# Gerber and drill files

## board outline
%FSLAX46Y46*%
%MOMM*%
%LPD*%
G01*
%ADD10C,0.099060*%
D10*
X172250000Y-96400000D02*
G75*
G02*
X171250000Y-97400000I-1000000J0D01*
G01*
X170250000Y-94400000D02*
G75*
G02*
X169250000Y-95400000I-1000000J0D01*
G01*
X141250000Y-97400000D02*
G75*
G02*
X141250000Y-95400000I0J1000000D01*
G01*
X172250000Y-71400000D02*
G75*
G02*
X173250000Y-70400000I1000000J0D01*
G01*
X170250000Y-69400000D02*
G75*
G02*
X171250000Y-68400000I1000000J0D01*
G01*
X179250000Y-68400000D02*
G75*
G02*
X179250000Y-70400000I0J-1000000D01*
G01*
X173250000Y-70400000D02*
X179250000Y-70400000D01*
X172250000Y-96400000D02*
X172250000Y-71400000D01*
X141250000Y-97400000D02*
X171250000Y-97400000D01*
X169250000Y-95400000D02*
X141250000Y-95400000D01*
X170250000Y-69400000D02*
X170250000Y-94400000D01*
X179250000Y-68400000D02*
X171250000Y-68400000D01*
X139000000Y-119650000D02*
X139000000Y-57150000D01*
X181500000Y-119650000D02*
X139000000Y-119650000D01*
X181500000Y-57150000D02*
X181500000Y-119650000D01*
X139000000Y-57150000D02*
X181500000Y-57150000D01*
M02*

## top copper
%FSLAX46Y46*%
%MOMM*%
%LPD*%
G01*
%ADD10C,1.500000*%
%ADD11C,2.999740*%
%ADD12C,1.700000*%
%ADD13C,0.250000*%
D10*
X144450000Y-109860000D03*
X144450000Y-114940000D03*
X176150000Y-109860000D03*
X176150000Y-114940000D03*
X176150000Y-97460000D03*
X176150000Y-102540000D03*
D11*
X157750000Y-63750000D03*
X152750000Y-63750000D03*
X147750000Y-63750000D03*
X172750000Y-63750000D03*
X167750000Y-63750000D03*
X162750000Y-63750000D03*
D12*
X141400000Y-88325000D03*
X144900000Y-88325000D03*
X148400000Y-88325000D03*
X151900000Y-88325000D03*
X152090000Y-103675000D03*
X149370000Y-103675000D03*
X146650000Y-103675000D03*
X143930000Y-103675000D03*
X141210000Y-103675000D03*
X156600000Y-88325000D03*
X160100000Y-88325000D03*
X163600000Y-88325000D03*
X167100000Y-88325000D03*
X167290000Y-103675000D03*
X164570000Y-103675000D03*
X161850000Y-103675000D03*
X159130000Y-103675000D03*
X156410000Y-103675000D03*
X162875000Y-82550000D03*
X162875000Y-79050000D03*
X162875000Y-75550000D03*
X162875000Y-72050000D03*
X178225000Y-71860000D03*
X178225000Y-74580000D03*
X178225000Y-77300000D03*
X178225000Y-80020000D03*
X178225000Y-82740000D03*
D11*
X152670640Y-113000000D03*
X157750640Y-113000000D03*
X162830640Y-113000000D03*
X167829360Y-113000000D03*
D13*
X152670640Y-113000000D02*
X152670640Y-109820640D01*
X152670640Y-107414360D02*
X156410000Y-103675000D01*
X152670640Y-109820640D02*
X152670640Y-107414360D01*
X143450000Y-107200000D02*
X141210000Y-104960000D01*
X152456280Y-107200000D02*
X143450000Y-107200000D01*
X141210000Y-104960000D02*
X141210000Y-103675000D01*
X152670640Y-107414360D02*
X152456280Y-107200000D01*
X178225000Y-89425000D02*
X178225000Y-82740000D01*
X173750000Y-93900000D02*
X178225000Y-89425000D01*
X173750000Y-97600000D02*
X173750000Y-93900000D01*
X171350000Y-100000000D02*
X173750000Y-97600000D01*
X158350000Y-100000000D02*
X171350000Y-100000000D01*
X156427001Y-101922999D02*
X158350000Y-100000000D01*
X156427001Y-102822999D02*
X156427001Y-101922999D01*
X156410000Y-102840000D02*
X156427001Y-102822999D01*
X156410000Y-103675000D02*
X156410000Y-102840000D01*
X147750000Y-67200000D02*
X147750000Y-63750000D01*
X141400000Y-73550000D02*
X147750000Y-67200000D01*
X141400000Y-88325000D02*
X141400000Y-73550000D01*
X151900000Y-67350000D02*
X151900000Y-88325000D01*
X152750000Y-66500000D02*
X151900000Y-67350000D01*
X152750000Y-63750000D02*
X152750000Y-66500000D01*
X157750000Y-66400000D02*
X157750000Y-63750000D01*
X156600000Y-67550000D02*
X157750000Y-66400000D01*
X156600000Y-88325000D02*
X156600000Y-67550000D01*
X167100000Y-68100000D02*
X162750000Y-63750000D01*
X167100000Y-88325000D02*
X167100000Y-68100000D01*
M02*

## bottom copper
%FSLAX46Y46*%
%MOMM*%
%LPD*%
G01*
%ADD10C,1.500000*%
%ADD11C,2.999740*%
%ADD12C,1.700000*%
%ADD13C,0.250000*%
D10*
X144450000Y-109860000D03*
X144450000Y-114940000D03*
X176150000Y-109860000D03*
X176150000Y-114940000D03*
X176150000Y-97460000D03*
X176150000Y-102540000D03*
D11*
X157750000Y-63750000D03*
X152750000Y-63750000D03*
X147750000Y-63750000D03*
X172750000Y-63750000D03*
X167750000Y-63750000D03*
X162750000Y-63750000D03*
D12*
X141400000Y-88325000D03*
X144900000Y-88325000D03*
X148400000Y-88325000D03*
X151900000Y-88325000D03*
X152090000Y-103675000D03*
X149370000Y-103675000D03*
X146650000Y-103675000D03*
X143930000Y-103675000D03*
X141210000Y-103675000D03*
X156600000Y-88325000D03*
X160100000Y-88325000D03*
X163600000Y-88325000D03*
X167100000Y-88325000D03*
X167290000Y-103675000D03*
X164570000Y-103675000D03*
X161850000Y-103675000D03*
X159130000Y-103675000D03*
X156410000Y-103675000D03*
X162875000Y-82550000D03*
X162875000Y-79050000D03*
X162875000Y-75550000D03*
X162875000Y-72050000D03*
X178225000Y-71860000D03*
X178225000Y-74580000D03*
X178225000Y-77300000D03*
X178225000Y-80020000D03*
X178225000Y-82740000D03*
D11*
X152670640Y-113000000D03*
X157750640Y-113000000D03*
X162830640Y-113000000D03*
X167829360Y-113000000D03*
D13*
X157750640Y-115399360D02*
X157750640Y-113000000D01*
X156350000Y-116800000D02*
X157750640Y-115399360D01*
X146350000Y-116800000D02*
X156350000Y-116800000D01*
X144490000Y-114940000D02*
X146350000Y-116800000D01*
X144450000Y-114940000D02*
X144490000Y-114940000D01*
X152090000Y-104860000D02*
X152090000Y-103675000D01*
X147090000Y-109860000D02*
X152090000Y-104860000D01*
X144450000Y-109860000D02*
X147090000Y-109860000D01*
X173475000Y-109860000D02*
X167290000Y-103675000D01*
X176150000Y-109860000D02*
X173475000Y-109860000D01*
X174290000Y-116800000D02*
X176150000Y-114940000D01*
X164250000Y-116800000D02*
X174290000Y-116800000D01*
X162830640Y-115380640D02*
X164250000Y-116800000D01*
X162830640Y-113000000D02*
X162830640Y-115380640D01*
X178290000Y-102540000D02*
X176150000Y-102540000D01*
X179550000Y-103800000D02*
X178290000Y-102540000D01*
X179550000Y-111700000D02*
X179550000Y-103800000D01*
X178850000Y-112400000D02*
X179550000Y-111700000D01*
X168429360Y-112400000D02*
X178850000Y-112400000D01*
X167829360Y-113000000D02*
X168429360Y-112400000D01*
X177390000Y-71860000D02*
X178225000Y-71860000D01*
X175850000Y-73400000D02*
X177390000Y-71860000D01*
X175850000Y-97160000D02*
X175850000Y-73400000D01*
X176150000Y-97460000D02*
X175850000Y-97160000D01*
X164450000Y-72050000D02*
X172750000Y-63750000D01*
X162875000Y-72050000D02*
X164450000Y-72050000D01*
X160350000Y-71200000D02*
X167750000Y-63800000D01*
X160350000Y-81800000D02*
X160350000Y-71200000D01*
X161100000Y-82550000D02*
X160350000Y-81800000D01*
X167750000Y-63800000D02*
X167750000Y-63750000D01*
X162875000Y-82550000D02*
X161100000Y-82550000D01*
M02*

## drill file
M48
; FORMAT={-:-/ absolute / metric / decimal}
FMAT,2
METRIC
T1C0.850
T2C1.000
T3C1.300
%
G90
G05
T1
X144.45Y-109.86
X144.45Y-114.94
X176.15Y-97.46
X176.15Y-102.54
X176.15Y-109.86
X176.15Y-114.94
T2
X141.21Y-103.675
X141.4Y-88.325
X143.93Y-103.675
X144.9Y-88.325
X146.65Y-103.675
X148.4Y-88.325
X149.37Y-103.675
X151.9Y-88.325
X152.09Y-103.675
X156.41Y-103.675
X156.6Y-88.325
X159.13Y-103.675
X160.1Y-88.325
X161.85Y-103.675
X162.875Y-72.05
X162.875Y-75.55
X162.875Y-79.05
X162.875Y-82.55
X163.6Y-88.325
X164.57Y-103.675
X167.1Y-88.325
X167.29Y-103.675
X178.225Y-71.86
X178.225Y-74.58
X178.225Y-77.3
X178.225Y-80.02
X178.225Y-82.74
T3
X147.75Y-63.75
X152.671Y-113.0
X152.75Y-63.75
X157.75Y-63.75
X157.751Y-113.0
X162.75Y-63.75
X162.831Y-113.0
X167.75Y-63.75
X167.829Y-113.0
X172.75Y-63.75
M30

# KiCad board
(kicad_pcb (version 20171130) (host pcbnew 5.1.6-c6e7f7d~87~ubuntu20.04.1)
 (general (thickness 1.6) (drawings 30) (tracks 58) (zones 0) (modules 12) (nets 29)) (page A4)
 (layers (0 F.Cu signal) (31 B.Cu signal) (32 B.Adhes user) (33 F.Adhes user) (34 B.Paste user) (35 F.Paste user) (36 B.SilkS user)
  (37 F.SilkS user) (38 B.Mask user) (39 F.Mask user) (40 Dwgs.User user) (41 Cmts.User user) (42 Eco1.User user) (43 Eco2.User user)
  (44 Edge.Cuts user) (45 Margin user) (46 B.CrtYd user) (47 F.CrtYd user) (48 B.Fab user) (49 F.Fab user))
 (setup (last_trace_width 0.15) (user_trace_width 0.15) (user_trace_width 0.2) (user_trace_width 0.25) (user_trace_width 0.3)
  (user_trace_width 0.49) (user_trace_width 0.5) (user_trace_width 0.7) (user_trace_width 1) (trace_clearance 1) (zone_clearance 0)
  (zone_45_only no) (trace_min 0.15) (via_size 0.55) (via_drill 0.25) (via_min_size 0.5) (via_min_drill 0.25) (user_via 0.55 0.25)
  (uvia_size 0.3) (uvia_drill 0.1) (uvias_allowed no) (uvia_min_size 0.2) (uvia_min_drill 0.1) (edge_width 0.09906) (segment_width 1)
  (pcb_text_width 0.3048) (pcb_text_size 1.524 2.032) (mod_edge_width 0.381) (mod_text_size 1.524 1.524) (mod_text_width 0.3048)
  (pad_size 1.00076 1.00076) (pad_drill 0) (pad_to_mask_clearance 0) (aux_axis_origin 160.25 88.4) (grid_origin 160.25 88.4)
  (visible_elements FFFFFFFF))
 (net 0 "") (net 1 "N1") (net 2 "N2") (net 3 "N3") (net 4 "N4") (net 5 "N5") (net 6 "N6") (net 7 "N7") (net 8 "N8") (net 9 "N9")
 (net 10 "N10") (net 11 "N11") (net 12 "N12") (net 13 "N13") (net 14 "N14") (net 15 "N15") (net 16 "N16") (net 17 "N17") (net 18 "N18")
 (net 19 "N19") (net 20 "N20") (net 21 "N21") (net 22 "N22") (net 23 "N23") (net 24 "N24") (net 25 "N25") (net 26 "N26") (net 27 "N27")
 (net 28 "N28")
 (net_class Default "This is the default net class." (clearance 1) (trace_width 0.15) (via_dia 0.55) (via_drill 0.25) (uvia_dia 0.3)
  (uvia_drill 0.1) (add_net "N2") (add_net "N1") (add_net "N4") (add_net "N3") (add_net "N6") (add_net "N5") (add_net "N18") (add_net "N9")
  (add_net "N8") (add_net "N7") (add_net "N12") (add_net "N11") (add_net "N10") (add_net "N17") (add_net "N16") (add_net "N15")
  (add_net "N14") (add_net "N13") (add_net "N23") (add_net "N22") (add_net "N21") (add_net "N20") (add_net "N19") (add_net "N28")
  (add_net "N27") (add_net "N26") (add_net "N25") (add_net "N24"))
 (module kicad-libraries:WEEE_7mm (layer B.Cu) (at 148.85 80.5 180)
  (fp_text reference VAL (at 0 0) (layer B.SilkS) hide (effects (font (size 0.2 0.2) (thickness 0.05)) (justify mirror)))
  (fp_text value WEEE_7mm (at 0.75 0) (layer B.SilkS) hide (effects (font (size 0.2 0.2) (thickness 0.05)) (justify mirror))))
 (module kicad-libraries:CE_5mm (layer B.Cu) (at 148.95 73.1 180)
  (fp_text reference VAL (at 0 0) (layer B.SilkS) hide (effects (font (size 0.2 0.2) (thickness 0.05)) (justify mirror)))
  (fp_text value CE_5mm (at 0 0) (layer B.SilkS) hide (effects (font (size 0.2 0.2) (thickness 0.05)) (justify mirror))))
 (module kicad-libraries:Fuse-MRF (layer F.Cu) (at 144.45 112.4 90)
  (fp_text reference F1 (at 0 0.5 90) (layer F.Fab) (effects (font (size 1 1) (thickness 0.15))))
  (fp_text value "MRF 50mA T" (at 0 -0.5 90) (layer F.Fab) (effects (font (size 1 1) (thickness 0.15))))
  (pad 2 thru_hole circle (at 2.54 0 90) (size 1.5 1.5) (drill 0.85) (layers *.Cu *.Mask) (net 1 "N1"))
  (pad 1 thru_hole circle (at -2.54 0 90) (size 1.5 1.5) (drill 0.85) (layers *.Cu *.Mask) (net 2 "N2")))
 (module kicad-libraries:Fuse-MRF (layer F.Cu) (at 176.15 112.4 90)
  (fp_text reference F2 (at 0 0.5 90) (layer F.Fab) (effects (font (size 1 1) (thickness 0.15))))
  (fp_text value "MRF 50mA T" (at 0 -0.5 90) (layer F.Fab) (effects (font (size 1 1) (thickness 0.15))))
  (pad 2 thru_hole circle (at 2.54 0 90) (size 1.5 1.5) (drill 0.85) (layers *.Cu *.Mask) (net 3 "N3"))
  (pad 1 thru_hole circle (at -2.54 0 90) (size 1.5 1.5) (drill 0.85) (layers *.Cu *.Mask) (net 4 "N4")))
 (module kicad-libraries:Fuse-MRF (layer F.Cu) (at 176.15 100 90)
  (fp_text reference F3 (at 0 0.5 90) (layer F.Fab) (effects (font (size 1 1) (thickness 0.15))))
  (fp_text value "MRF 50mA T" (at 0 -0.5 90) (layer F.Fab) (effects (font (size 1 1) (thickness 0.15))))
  (pad 2 thru_hole circle (at 2.54 0 90) (size 1.5 1.5) (drill 0.85) (layers *.Cu *.Mask) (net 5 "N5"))
  (pad 1 thru_hole circle (at -2.54 0 90) (size 1.5 1.5) (drill 0.85) (layers *.Cu *.Mask) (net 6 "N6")))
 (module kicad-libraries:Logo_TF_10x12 (layer F.Cu) (at 149.25 74.4)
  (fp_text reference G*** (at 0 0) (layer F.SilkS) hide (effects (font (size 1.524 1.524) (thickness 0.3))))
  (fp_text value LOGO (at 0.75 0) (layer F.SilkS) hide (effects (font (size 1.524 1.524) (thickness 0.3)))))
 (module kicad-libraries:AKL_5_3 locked (layer F.Cu) (at 152.75 63.75)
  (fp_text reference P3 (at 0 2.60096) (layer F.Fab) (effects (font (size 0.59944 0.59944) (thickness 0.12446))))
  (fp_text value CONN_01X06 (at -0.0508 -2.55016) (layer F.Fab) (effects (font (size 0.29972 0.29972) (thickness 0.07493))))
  (pad 3 thru_hole circle (at 5 0) (size 2.99974 2.99974) (drill 1.30048) (layers *.Cu *.Mask F.SilkS) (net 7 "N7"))
  (pad 2 thru_hole circle (at 0 0) (size 2.99974 2.99974) (drill 1.30048) (layers *.Cu *.Mask F.SilkS) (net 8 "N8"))
  (pad 1 thru_hole circle (at -5 0) (size 2.99974 2.99974) (drill 1.30048) (layers *.Cu *.Mask F.SilkS) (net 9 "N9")))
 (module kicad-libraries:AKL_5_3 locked (layer F.Cu) (at 167.75 63.75)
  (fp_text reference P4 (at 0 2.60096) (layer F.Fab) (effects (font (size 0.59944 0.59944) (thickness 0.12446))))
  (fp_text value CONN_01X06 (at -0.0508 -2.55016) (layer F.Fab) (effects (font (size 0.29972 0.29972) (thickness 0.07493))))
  (pad 3 thru_hole circle (at 5 0) (size 2.99974 2.99974) (drill 1.30048) (layers *.Cu *.Mask F.SilkS) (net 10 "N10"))
  (pad 2 thru_hole circle (at 0 0) (size 2.99974 2.99974) (drill 1.30048) (layers *.Cu *.Mask F.SilkS) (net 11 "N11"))
  (pad 1 thru_hole circle (at -5 0) (size 2.99974 2.99974) (drill 1.30048) (layers *.Cu *.Mask F.SilkS) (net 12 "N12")))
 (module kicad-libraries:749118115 (layer F.Cu) (at 146.65 96)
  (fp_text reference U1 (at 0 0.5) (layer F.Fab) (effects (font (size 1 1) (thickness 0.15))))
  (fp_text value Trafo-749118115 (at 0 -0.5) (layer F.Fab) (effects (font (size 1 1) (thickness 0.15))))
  (pad 9 thru_hole circle (at -5.25 -7.675) (size 1.7 1.7) (drill 1) (layers *.Cu *.Mask) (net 9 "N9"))
  (pad 8 thru_hole circle (at -1.75 -7.675) (size 1.7 1.7) (drill 1) (layers *.Cu *.Mask) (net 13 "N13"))
  (pad 7 thru_hole circle (at 1.75 -7.675) (size 1.7 1.7) (drill 1) (layers *.Cu *.Mask) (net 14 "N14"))
  (pad 6 thru_hole circle (at 5.25 -7.675) (size 1.7 1.7) (drill 1) (layers *.Cu *.Mask) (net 8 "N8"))
  (pad 5 thru_hole circle (at 5.44 7.675) (size 1.7 1.7) (drill 1) (layers *.Cu *.Mask) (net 1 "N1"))
  (pad 4 thru_hole circle (at 2.72 7.675) (size 1.7 1.7) (drill 1) (layers *.Cu *.Mask) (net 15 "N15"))
  (pad 3 thru_hole circle (at 0 7.675) (size 1.7 1.7) (drill 1) (layers *.Cu *.Mask) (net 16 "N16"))
  (pad 2 thru_hole circle (at -2.72 7.675) (size 1.7 1.7) (drill 1) (layers *.Cu *.Mask) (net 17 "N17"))
  (pad 1 thru_hole circle (at -5.44 7.675) (size 1.7 1.7) (drill 1) (layers *.Cu *.Mask) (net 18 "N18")))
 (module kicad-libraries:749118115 (layer F.Cu) (at 161.85 96)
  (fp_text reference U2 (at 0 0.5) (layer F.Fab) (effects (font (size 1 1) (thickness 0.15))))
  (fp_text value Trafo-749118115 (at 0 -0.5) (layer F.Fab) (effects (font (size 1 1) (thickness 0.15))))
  (pad 9 thru_hole circle (at -5.25 -7.675) (size 1.7 1.7) (drill 1) (layers *.Cu *.Mask) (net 7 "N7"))
  (pad 8 thru_hole circle (at -1.75 -7.675) (size 1.7 1.7) (drill 1) (layers *.Cu *.Mask) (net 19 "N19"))
  (pad 7 thru_hole circle (at 1.75 -7.675) (size 1.7 1.7) (drill 1) (layers *.Cu *.Mask) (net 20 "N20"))
  (pad 6 thru_hole circle (at 5.25 -7.675) (size 1.7 1.7) (drill 1) (layers *.Cu *.Mask) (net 12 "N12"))
  (pad 5 thru_hole circle (at 5.44 7.675) (size 1.7 1.7) (drill 1) (layers *.Cu *.Mask) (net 3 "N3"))
  (pad 4 thru_hole circle (at 2.72 7.675) (size 1.7 1.7) (drill 1) (layers *.Cu *.Mask) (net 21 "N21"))
  (pad 3 thru_hole circle (at 0 7.675) (size 1.7 1.7) (drill 1) (layers *.Cu *.Mask) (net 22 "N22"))
  (pad 2 thru_hole circle (at -2.72 7.675) (size 1.7 1.7) (drill 1) (layers *.Cu *.Mask) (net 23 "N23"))
  (pad 1 thru_hole circle (at -5.44 7.675) (size 1.7 1.7) (drill 1) (layers *.Cu *.Mask) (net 18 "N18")))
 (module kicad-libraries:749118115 (layer F.Cu) (at 170.55 77.3 90)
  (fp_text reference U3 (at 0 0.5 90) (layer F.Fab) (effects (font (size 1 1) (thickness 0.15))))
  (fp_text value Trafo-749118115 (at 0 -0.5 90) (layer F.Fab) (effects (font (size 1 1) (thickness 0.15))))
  (pad 9 thru_hole circle (at -5.25 -7.675 90) (size 1.7 1.7) (drill 1) (layers *.Cu *.Mask) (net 11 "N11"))
  (pad 8 thru_hole circle (at -1.75 -7.675 90) (size 1.7 1.7) (drill 1) (layers *.Cu *.Mask) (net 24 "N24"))
  (pad 7 thru_hole circle (at 1.75 -7.675 90) (size 1.7 1.7) (drill 1) (layers *.Cu *.Mask) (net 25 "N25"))
  (pad 6 thru_hole circle (at 5.25 -7.675 90) (size 1.7 1.7) (drill 1) (layers *.Cu *.Mask) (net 10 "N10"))
  (pad 5 thru_hole circle (at 5.44 7.675 90) (size 1.7 1.7) (drill 1) (layers *.Cu *.Mask) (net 5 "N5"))
  (pad 4 thru_hole circle (at 2.72 7.675 90) (size 1.7 1.7) (drill 1) (layers *.Cu *.Mask) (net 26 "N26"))
  (pad 3 thru_hole circle (at 0 7.675 90) (size 1.7 1.7) (drill 1) (layers *.Cu *.Mask) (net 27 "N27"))
  (pad 2 thru_hole circle (at -2.72 7.675 90) (size 1.7 1.7) (drill 1) (layers *.Cu *.Mask) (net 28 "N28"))
  (pad 1 thru_hole circle (at -5.44 7.675 90) (size 1.7 1.7) (drill 1) (layers *.Cu *.Mask) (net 18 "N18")))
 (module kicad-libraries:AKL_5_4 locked (layer F.Cu) (at 160.25 113 180)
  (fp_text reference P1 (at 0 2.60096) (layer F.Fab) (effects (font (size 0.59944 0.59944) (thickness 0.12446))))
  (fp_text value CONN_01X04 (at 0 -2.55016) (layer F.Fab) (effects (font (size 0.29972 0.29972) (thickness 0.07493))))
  (pad 1 thru_hole circle (at 7.57936 0 180) (size 2.99974 2.99974) (drill 1.30048) (layers *.Cu *.Mask F.SilkS) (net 18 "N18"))
  (pad 2 thru_hole circle (at 2.49936 0 180) (size 2.99974 2.99974) (drill 1.30048) (layers *.Cu *.Mask F.SilkS) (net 2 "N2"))
  (pad 3 thru_hole circle (at -2.58064 0 180) (size 2.99974 2.99974) (drill 1.30048) (layers *.Cu *.Mask F.SilkS) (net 4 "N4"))
  (pad 4 thru_hole circle (at -7.57936 0 180) (size 2.99974 2.99974) (drill 1.30048) (layers *.Cu *.Mask F.SilkS) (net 6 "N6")))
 (gr_arc (start 171.25 96.4) (end 171.25 97.4) (angle -90) (layer Edge.Cuts) (width 0.09906))
 (gr_arc (start 169.25 94.4) (end 169.25 95.4) (angle -90) (layer Edge.Cuts) (width 0.09906))
 (gr_arc (start 141.25 96.4) (end 141.25 95.4) (angle -180) (layer Edge.Cuts) (width 0.09906))
 (gr_arc (start 173.25 71.4) (end 173.25 70.4) (angle -90) (layer Edge.Cuts) (width 0.09906))
 (gr_arc (start 171.25 69.4) (end 171.25 68.4) (angle -90) (layer Edge.Cuts) (width 0.09906))
 (gr_arc (start 179.25 69.4) (end 179.25 70.4) (angle -180) (layer Edge.Cuts) (width 0.09906))
 (gr_line (start 173.25 70.4) (end 179.25 70.4) (layer Edge.Cuts) (width 0.09906))
 (gr_line (start 172.25 96.4) (end 172.25 71.4) (layer Edge.Cuts) (width 0.09906))
 (gr_line (start 141.25 97.4) (end 171.25 97.4) (layer Edge.Cuts) (width 0.09906))
 (gr_line (start 169.25 95.4) (end 141.25 95.4) (layer Edge.Cuts) (width 0.09906))
 (gr_line (start 170.25 69.4) (end 170.25 94.4) (layer Edge.Cuts) (width 0.09906))
 (gr_line (start 179.25 68.4) (end 171.25 68.4) (layer Edge.Cuts) (width 0.09906))
 (gr_line (start 139 119.65) (end 139 57.15) (layer Edge.Cuts) (width 0.09906))
 (gr_line (start 181.5 119.65) (end 139 119.65) (layer Edge.Cuts) (width 0.09906))
 (gr_line (start 181.5 57.15) (end 181.5 119.65) (layer Edge.Cuts) (width 0.09906))
 (gr_line (start 139 57.15) (end 181.5 57.15) (layer Edge.Cuts) (width 0.09906))
 (segment (start 157.75064 115.39936) (end 157.75064 113) (width 0.25) (layer B.Cu) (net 2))
 (segment (start 156.35 116.8) (end 157.75064 115.39936) (width 0.25) (layer B.Cu) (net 2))
 (segment (start 146.35 116.8) (end 156.35 116.8) (width 0.25) (layer B.Cu) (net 2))
 (segment (start 144.49 114.94) (end 146.35 116.8) (width 0.25) (layer B.Cu) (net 2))
 (segment (start 144.45 114.94) (end 144.49 114.94) (width 0.25) (layer B.Cu) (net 2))
 (segment (start 152.09 104.86) (end 152.09 103.675) (width 0.25) (layer B.Cu) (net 1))
 (segment (start 147.09 109.86) (end 152.09 104.86) (width 0.25) (layer B.Cu) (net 1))
 (segment (start 144.45 109.86) (end 147.09 109.86) (width 0.25) (layer B.Cu) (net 1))
 (segment (start 173.475 109.86) (end 167.29 103.675) (width 0.25) (layer B.Cu) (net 3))
 (segment (start 176.15 109.86) (end 173.475 109.86) (width 0.25) (layer B.Cu) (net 3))
 (segment (start 174.29 116.8) (end 176.15 114.94) (width 0.25) (layer B.Cu) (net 4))
 (segment (start 164.25 116.8) (end 174.29 116.8) (width 0.25) (layer B.Cu) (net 4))
 (segment (start 162.83064 115.38064) (end 164.25 116.8) (width 0.25) (layer B.Cu) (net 4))
 (segment (start 162.83064 113) (end 162.83064 115.38064) (width 0.25) (layer B.Cu) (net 4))
 (segment (start 178.29 102.54) (end 176.15 102.54) (width 0.25) (layer B.Cu) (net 6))
 (segment (start 179.55 103.8) (end 178.29 102.54) (width 0.25) (layer B.Cu) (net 6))
 (segment (start 179.55 111.7) (end 179.55 103.8) (width 0.25) (layer B.Cu) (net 6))
 (segment (start 178.85 112.4) (end 179.55 111.7) (width 0.25) (layer B.Cu) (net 6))
 (segment (start 168.42936 112.4) (end 178.85 112.4) (width 0.25) (layer B.Cu) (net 6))
 (segment (start 167.82936 113) (end 168.42936 112.4) (width 0.25) (layer B.Cu) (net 6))
 (segment (start 177.39 71.86) (end 178.225 71.86) (width 0.25) (layer B.Cu) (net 5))
 (segment (start 175.85 73.4) (end 177.39 71.86) (width 0.25) (layer B.Cu) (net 5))
 (segment (start 175.85 97.16) (end 175.85 73.4) (width 0.25) (layer B.Cu) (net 5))
 (segment (start 176.15 97.46) (end 175.85 97.16) (width 0.25) (layer B.Cu) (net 5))
 (segment (start 152.67064 113) (end 152.67064 109.82064) (width 0.25) (layer F.Cu) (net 18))
 (segment (start 152.67064 107.41436) (end 156.41 103.675) (width 0.25) (layer F.Cu) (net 18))
 (segment (start 152.67064 109.82064) (end 152.67064 107.41436) (width 0.25) (layer F.Cu) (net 18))
 (segment (start 143.45 107.2) (end 141.21 104.96) (width 0.25) (layer F.Cu) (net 18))
 (segment (start 152.45628 107.2) (end 143.45 107.2) (width 0.25) (layer F.Cu) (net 18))
 (segment (start 141.21 104.96) (end 141.21 103.675) (width 0.25) (layer F.Cu) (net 18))
 (segment (start 152.67064 107.41436) (end 152.45628 107.2) (width 0.25) (layer F.Cu) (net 18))
 (segment (start 178.225 89.425) (end 178.225 82.74) (width 0.25) (layer F.Cu) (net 18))
 (segment (start 173.75 93.9) (end 178.225 89.425) (width 0.25) (layer F.Cu) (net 18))
 (segment (start 173.75 97.6) (end 173.75 93.9) (width 0.25) (layer F.Cu) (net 18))
 (segment (start 171.35 100) (end 173.75 97.6) (width 0.25) (layer F.Cu) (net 18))
 (segment (start 158.35 100) (end 171.35 100) (width 0.25) (layer F.Cu) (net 18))
 (segment (start 156.427001 101.922999) (end 158.35 100) (width 0.25) (layer F.Cu) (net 18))
 (segment (start 156.427001 102.822999) (end 156.427001 101.922999) (width 0.25) (layer F.Cu) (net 18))
 (segment (start 156.41 102.84) (end 156.427001 102.822999) (width 0.25) (layer F.Cu) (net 18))
 (segment (start 156.41 103.675) (end 156.41 102.84) (width 0.25) (layer F.Cu) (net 18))
 (segment (start 147.75 67.2) (end 147.75 63.75) (width 0.25) (layer F.Cu) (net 9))
 (segment (start 141.4 73.55) (end 147.75 67.2) (width 0.25) (layer F.Cu) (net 9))
 (segment (start 141.4 88.325) (end 141.4 73.55) (width 0.25) (layer F.Cu) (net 9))
 (segment (start 151.9 67.35) (end 151.9 88.325) (width 0.25) (layer F.Cu) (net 8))
 (segment (start 152.75 66.5) (end 151.9 67.35) (width 0.25) (layer F.Cu) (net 8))
 (segment (start 152.75 63.75) (end 152.75 66.5) (width 0.25) (layer F.Cu) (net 8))
 (segment (start 157.75 66.4) (end 157.75 63.75) (width 0.25) (layer F.Cu) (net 7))
 (segment (start 156.6 67.55) (end 157.75 66.4) (width 0.25) (layer F.Cu) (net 7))
 (segment (start 156.6 88.325) (end 156.6 67.55) (width 0.25) (layer F.Cu) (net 7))
 (segment (start 164.45 72.05) (end 172.75 63.75) (width 0.25) (layer B.Cu) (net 10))
 (segment (start 162.875 72.05) (end 164.45 72.05) (width 0.25) (layer B.Cu) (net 10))
 (segment (start 160.35 71.2) (end 167.75 63.8) (width 0.25) (layer B.Cu) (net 11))
 (segment (start 160.35 81.8) (end 160.35 71.2) (width 0.25) (layer B.Cu) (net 11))
 (segment (start 161.1 82.55) (end 160.35 81.8) (width 0.25) (layer B.Cu) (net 11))
 (segment (start 167.75 63.8) (end 167.75 63.75) (width 0.25) (layer B.Cu) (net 11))
 (segment (start 162.875 82.55) (end 161.1 82.55) (width 0.25) (layer B.Cu) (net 11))
 (segment (start 167.1 68.1) (end 162.75 63.75) (width 0.25) (layer F.Cu) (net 12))
 (segment (start 167.1 88.325) (end 167.1 68.1) (width 0.25) (layer F.Cu) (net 12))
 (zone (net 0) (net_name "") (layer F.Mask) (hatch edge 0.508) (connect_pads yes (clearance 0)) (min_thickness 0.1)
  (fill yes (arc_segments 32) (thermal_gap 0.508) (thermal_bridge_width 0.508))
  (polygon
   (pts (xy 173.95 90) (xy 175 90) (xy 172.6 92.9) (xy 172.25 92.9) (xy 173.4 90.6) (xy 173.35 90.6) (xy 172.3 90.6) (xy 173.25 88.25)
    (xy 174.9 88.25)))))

